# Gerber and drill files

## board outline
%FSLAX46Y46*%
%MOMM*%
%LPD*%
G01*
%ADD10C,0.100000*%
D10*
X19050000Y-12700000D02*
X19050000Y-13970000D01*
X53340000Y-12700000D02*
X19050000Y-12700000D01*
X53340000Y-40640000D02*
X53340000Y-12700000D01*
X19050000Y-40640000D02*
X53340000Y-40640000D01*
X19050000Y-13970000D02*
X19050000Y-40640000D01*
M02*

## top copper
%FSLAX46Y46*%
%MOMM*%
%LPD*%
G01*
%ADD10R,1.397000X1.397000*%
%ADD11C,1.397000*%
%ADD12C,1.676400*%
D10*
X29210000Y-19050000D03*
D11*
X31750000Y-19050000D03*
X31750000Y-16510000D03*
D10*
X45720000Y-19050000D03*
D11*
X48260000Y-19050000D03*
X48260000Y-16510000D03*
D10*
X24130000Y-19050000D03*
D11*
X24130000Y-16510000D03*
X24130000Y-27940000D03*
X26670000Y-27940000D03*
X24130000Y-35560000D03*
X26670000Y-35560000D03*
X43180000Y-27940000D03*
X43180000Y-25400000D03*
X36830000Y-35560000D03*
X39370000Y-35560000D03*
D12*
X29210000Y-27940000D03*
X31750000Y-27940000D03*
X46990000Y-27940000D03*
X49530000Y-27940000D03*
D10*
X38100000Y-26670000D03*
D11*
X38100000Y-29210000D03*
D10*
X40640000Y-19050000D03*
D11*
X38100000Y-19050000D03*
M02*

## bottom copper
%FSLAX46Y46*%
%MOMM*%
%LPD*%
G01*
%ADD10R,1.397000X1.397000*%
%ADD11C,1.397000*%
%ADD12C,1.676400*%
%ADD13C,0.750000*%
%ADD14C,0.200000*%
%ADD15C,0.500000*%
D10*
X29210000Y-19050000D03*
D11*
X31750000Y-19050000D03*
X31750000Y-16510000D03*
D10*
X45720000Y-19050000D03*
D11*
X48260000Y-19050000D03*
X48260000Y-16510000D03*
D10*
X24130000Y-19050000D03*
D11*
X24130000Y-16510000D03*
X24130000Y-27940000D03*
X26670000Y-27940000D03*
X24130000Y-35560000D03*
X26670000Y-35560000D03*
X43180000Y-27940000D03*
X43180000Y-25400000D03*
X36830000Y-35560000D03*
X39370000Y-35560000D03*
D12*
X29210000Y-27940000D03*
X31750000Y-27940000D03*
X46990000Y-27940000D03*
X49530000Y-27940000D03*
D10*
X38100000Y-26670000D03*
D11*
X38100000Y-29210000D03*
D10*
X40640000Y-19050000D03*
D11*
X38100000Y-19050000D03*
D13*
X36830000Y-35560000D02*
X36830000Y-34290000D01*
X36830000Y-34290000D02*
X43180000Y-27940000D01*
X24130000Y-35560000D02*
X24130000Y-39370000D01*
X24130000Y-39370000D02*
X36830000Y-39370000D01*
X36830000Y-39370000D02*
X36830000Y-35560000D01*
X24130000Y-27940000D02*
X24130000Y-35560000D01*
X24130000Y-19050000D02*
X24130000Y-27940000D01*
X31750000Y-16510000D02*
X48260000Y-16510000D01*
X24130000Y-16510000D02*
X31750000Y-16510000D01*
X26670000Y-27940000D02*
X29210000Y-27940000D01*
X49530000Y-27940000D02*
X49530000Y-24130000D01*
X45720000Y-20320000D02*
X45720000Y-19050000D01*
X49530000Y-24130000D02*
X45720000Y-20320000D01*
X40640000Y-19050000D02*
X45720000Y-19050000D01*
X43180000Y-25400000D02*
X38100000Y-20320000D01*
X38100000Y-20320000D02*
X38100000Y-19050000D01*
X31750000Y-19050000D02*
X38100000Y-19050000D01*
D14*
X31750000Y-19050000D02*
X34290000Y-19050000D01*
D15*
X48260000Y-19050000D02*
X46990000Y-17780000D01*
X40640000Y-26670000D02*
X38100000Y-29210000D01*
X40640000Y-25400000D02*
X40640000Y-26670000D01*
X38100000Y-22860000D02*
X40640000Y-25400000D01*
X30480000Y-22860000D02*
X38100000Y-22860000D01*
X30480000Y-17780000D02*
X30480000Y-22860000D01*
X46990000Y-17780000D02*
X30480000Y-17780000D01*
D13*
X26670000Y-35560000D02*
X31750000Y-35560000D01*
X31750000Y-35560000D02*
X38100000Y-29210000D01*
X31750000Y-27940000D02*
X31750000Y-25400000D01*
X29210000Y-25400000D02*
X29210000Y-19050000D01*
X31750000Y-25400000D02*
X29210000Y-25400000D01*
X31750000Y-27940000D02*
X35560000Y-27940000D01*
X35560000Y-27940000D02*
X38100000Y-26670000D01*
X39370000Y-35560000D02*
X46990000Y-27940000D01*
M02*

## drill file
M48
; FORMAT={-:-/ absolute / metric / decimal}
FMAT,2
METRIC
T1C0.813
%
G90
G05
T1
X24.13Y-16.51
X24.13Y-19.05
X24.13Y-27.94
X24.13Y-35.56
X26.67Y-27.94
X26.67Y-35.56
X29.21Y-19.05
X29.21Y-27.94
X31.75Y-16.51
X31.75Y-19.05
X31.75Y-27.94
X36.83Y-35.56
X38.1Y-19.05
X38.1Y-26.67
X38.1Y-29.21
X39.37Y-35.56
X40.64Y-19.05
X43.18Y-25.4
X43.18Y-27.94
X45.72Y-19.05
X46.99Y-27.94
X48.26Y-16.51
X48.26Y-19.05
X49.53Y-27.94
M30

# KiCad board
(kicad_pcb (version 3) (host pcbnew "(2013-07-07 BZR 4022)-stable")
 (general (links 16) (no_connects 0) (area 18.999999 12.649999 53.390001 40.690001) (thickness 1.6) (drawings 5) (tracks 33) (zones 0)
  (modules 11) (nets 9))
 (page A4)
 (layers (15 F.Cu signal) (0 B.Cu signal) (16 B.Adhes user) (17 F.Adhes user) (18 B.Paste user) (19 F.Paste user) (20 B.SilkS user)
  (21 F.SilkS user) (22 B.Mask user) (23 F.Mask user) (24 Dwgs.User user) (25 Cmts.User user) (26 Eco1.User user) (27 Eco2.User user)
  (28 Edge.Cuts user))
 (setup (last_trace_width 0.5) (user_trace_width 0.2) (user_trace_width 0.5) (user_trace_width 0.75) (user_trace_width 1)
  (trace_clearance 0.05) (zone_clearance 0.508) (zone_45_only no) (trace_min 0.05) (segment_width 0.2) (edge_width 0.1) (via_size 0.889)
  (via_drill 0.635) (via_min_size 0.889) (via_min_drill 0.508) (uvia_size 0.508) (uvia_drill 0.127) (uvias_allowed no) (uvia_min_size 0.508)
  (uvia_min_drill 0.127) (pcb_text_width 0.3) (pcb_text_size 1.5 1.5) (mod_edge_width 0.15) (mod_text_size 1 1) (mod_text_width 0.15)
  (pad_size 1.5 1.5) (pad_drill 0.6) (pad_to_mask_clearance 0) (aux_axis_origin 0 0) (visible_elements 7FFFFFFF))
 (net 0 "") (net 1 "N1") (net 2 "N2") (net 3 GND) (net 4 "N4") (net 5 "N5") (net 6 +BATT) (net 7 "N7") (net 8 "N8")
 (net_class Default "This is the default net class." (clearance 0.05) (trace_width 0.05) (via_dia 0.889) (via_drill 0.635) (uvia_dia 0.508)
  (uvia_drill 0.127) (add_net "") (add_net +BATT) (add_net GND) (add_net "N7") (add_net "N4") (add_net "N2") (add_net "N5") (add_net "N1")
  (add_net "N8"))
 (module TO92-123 (layer F.Cu) (at 30.48 17.78 180)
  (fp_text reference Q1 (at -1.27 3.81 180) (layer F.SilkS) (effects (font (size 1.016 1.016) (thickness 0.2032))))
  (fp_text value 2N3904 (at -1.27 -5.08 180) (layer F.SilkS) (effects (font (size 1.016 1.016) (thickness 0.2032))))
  (pad 3 thru_hole rect (at 1.27 -1.27 180) (size 1.397 1.397) (drill 0.8128) (layers *.Cu *.Mask F.SilkS) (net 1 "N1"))
  (pad 2 thru_hole circle (at -1.27 -1.27 180) (size 1.397 1.397) (drill 0.8128) (layers *.Cu *.Mask F.SilkS) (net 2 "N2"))
  (pad 1 thru_hole circle (at -1.27 1.27 180) (size 1.397 1.397) (drill 0.8128) (layers *.Cu *.Mask F.SilkS) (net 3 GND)))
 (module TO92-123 (layer F.Cu) (at 46.99 17.78 180)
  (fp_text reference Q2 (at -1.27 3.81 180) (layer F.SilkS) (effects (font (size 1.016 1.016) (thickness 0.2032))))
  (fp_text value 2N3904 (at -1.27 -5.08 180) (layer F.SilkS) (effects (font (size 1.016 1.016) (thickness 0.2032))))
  (pad 3 thru_hole rect (at 1.27 -1.27 180) (size 1.397 1.397) (drill 0.8128) (layers *.Cu *.Mask F.SilkS) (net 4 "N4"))
  (pad 2 thru_hole circle (at -1.27 -1.27 180) (size 1.397 1.397) (drill 0.8128) (layers *.Cu *.Mask F.SilkS) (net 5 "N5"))
  (pad 1 thru_hole circle (at -1.27 1.27 180) (size 1.397 1.397) (drill 0.8128) (layers *.Cu *.Mask F.SilkS) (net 3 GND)))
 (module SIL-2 (layer F.Cu) (at 24.13 17.78 90)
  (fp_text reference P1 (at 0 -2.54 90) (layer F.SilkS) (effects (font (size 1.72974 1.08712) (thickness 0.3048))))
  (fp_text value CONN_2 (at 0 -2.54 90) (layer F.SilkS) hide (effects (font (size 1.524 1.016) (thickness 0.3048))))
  (pad 1 thru_hole rect (at -1.27 0 90) (size 1.397 1.397) (drill 0.8128) (layers *.Cu *.Mask F.SilkS) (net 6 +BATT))
  (pad 2 thru_hole circle (at 1.27 0 90) (size 1.397 1.397) (drill 0.8128) (layers *.Cu *.Mask F.SilkS) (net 3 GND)))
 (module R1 (layer F.Cu) (at 25.4 27.94) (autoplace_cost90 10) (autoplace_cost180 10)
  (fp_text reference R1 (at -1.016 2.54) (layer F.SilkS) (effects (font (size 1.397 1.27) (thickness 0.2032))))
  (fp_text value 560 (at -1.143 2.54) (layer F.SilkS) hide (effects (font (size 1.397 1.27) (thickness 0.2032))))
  (pad 1 thru_hole circle (at -1.27 0) (size 1.397 1.397) (drill 0.8128) (layers *.Cu *.Mask F.SilkS) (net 6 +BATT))
  (pad 2 thru_hole circle (at 1.27 0) (size 1.397 1.397) (drill 0.8128) (layers *.Cu *.Mask F.SilkS) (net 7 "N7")))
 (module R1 (layer F.Cu) (at 25.4 35.56) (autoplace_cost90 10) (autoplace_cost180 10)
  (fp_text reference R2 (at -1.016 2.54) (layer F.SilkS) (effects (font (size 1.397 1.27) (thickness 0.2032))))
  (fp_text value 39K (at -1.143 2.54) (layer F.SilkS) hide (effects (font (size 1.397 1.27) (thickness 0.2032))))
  (pad 1 thru_hole circle (at -1.27 0) (size 1.397 1.397) (drill 0.8128) (layers *.Cu *.Mask F.SilkS) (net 6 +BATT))
  (pad 2 thru_hole circle (at 1.27 0) (size 1.397 1.397) (drill 0.8128) (layers *.Cu *.Mask F.SilkS) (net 5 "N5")))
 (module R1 (layer F.Cu) (at 43.18 26.67 90) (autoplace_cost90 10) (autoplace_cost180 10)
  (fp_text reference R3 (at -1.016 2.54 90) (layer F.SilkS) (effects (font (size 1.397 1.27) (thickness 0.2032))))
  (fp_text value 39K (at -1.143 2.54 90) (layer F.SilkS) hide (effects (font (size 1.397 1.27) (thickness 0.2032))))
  (pad 1 thru_hole circle (at -1.27 0 90) (size 1.397 1.397) (drill 0.8128) (layers *.Cu *.Mask F.SilkS) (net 6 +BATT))
  (pad 2 thru_hole circle (at 1.27 0 90) (size 1.397 1.397) (drill 0.8128) (layers *.Cu *.Mask F.SilkS) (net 2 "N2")))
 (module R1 (layer F.Cu) (at 38.1 35.56) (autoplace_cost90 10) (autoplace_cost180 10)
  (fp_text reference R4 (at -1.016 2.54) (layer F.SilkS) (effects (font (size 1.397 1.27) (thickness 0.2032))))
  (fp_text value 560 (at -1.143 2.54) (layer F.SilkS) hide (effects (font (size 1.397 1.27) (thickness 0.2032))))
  (pad 1 thru_hole circle (at -1.27 0) (size 1.397 1.397) (drill 0.8128) (layers *.Cu *.Mask F.SilkS) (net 6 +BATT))
  (pad 2 thru_hole circle (at 1.27 0) (size 1.397 1.397) (drill 0.8128) (layers *.Cu *.Mask F.SilkS) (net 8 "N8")))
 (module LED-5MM (layer F.Cu) (at 30.48 27.94)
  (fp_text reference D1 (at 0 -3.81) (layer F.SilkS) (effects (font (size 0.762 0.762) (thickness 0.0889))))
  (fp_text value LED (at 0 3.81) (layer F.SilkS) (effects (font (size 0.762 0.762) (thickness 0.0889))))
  (pad 1 thru_hole circle (at -1.27 0) (size 1.6764 1.6764) (drill 0.8128) (layers *.Cu *.Mask F.SilkS) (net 7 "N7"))
  (pad 2 thru_hole circle (at 1.27 0) (size 1.6764 1.6764) (drill 0.8128) (layers *.Cu *.Mask F.SilkS) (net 1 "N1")))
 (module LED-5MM (layer F.Cu) (at 48.26 27.94)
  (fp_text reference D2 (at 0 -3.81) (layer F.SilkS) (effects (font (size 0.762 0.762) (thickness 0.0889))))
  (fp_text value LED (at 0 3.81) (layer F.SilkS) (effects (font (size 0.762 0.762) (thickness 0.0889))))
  (pad 1 thru_hole circle (at -1.27 0) (size 1.6764 1.6764) (drill 0.8128) (layers *.Cu *.Mask F.SilkS) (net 8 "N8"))
  (pad 2 thru_hole circle (at 1.27 0) (size 1.6764 1.6764) (drill 0.8128) (layers *.Cu *.Mask F.SilkS) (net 4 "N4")))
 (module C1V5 (layer F.Cu) (at 38.1 27.94 270)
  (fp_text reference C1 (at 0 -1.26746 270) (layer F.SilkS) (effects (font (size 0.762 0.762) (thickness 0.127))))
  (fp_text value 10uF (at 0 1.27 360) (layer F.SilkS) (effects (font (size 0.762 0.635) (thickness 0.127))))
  (pad 1 thru_hole rect (at -1.27 0 270) (size 1.397 1.397) (drill 0.8128) (layers *.Cu *.Mask F.SilkS) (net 1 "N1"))
  (pad 2 thru_hole circle (at 1.27 0 270) (size 1.397 1.397) (drill 0.8128) (layers *.Cu *.Mask F.SilkS) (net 5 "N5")))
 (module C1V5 (layer F.Cu) (at 39.37 19.05 180)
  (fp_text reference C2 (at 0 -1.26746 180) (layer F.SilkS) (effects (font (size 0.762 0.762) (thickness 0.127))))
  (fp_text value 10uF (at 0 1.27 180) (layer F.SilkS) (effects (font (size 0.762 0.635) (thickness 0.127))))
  (pad 1 thru_hole rect (at -1.27 0 180) (size 1.397 1.397) (drill 0.8128) (layers *.Cu *.Mask F.SilkS) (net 4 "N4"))
  (pad 2 thru_hole circle (at 1.27 0 180) (size 1.397 1.397) (drill 0.8128) (layers *.Cu *.Mask F.SilkS) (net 2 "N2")))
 (gr_line (start 19.05 12.7) (end 19.05 13.97) (angle 90) (layer Edge.Cuts) (width 0.1))
 (gr_line (start 53.34 12.7) (end 19.05 12.7) (angle 90) (layer Edge.Cuts) (width 0.1))
 (gr_line (start 53.34 40.64) (end 53.34 12.7) (angle 90) (layer Edge.Cuts) (width 0.1))
 (gr_line (start 19.05 40.64) (end 53.34 40.64) (angle 90) (layer Edge.Cuts) (width 0.1))
 (gr_line (start 19.05 13.97) (end 19.05 40.64) (angle 90) (layer Edge.Cuts) (width 0.1))
 (segment (start 36.83 35.56) (end 36.83 34.29) (width 0.75) (layer B.Cu) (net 6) (status 10))
 (segment (start 36.83 34.29) (end 43.18 27.94) (width 0.75) (layer B.Cu) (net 6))
 (segment (start 24.13 35.56) (end 24.13 39.37) (width 0.75) (layer B.Cu) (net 6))
 (segment (start 24.13 39.37) (end 36.83 39.37) (width 0.75) (layer B.Cu) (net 6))
 (segment (start 36.83 39.37) (end 36.83 35.56) (width 0.75) (layer B.Cu) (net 6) (status 20))
 (segment (start 24.13 27.94) (end 24.13 35.56) (width 0.75) (layer B.Cu) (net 6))
 (segment (start 24.13 19.05) (end 24.13 27.94) (width 0.75) (layer B.Cu) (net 6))
 (segment (start 31.75 16.51) (end 48.26 16.51) (width 0.75) (layer B.Cu) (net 3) (status 10))
 (segment (start 24.13 16.51) (end 31.75 16.51) (width 0.75) (layer B.Cu) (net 3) (status 20))
 (segment (start 26.67 27.94) (end 29.21 27.94) (width 0.75) (layer B.Cu) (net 7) (status 20))
 (segment (start 49.53 27.94) (end 49.53 24.13) (width 0.75) (layer B.Cu) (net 4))
 (segment (start 45.72 20.32) (end 45.72 19.05) (width 0.75) (layer B.Cu) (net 4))
 (segment (start 49.53 24.13) (end 45.72 20.32) (width 0.75) (layer B.Cu) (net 4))
 (segment (start 40.64 19.05) (end 45.72 19.05) (width 0.75) (layer B.Cu) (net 4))
 (segment (start 43.18 25.4) (end 38.1 20.32) (width 0.75) (layer B.Cu) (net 2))
 (segment (start 38.1 20.32) (end 38.1 19.05) (width 0.75) (layer B.Cu) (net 2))
 (segment (start 31.75 19.05) (end 38.1 19.05) (width 0.75) (layer B.Cu) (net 2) (status 10))
 (segment (start 31.75 19.05) (end 34.29 19.05) (width 0.2) (layer B.Cu) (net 2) (status 10))
 (segment (start 48.26 19.05) (end 46.99 17.78) (width 0.5) (layer B.Cu) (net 5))
 (segment (start 40.64 26.67) (end 38.1 29.21) (width 0.5) (layer B.Cu) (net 5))
 (segment (start 40.64 25.4) (end 40.64 26.67) (width 0.5) (layer B.Cu) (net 5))
 (segment (start 38.1 22.86) (end 40.64 25.4) (width 0.5) (layer B.Cu) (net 5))
 (segment (start 30.48 22.86) (end 38.1 22.86) (width 0.5) (layer B.Cu) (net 5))
 (segment (start 30.48 17.78) (end 30.48 22.86) (width 0.5) (layer B.Cu) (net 5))
 (segment (start 46.99 17.78) (end 30.48 17.78) (width 0.5) (layer B.Cu) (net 5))
 (segment (start 26.67 35.56) (end 31.75 35.56) (width 0.75) (layer B.Cu) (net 5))
 (segment (start 31.75 35.56) (end 38.1 29.21) (width 0.75) (layer B.Cu) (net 5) (status 20))
 (segment (start 31.75 27.94) (end 31.75 25.4) (width 0.75) (layer B.Cu) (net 1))
 (segment (start 29.21 25.4) (end 29.21 19.05) (width 0.75) (layer B.Cu) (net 1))
 (segment (start 31.75 25.4) (end 29.21 25.4) (width 0.75) (layer B.Cu) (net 1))
 (segment (start 31.75 27.94) (end 35.56 27.94) (width 0.75) (layer B.Cu) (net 1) (status 10))
 (segment (start 35.56 27.94) (end 38.1 26.67) (width 0.75) (layer B.Cu) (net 1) (status 20))
 (segment (start 39.37 35.56) (end 46.99 27.94) (width 0.75) (layer B.Cu) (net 8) (status 10)))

